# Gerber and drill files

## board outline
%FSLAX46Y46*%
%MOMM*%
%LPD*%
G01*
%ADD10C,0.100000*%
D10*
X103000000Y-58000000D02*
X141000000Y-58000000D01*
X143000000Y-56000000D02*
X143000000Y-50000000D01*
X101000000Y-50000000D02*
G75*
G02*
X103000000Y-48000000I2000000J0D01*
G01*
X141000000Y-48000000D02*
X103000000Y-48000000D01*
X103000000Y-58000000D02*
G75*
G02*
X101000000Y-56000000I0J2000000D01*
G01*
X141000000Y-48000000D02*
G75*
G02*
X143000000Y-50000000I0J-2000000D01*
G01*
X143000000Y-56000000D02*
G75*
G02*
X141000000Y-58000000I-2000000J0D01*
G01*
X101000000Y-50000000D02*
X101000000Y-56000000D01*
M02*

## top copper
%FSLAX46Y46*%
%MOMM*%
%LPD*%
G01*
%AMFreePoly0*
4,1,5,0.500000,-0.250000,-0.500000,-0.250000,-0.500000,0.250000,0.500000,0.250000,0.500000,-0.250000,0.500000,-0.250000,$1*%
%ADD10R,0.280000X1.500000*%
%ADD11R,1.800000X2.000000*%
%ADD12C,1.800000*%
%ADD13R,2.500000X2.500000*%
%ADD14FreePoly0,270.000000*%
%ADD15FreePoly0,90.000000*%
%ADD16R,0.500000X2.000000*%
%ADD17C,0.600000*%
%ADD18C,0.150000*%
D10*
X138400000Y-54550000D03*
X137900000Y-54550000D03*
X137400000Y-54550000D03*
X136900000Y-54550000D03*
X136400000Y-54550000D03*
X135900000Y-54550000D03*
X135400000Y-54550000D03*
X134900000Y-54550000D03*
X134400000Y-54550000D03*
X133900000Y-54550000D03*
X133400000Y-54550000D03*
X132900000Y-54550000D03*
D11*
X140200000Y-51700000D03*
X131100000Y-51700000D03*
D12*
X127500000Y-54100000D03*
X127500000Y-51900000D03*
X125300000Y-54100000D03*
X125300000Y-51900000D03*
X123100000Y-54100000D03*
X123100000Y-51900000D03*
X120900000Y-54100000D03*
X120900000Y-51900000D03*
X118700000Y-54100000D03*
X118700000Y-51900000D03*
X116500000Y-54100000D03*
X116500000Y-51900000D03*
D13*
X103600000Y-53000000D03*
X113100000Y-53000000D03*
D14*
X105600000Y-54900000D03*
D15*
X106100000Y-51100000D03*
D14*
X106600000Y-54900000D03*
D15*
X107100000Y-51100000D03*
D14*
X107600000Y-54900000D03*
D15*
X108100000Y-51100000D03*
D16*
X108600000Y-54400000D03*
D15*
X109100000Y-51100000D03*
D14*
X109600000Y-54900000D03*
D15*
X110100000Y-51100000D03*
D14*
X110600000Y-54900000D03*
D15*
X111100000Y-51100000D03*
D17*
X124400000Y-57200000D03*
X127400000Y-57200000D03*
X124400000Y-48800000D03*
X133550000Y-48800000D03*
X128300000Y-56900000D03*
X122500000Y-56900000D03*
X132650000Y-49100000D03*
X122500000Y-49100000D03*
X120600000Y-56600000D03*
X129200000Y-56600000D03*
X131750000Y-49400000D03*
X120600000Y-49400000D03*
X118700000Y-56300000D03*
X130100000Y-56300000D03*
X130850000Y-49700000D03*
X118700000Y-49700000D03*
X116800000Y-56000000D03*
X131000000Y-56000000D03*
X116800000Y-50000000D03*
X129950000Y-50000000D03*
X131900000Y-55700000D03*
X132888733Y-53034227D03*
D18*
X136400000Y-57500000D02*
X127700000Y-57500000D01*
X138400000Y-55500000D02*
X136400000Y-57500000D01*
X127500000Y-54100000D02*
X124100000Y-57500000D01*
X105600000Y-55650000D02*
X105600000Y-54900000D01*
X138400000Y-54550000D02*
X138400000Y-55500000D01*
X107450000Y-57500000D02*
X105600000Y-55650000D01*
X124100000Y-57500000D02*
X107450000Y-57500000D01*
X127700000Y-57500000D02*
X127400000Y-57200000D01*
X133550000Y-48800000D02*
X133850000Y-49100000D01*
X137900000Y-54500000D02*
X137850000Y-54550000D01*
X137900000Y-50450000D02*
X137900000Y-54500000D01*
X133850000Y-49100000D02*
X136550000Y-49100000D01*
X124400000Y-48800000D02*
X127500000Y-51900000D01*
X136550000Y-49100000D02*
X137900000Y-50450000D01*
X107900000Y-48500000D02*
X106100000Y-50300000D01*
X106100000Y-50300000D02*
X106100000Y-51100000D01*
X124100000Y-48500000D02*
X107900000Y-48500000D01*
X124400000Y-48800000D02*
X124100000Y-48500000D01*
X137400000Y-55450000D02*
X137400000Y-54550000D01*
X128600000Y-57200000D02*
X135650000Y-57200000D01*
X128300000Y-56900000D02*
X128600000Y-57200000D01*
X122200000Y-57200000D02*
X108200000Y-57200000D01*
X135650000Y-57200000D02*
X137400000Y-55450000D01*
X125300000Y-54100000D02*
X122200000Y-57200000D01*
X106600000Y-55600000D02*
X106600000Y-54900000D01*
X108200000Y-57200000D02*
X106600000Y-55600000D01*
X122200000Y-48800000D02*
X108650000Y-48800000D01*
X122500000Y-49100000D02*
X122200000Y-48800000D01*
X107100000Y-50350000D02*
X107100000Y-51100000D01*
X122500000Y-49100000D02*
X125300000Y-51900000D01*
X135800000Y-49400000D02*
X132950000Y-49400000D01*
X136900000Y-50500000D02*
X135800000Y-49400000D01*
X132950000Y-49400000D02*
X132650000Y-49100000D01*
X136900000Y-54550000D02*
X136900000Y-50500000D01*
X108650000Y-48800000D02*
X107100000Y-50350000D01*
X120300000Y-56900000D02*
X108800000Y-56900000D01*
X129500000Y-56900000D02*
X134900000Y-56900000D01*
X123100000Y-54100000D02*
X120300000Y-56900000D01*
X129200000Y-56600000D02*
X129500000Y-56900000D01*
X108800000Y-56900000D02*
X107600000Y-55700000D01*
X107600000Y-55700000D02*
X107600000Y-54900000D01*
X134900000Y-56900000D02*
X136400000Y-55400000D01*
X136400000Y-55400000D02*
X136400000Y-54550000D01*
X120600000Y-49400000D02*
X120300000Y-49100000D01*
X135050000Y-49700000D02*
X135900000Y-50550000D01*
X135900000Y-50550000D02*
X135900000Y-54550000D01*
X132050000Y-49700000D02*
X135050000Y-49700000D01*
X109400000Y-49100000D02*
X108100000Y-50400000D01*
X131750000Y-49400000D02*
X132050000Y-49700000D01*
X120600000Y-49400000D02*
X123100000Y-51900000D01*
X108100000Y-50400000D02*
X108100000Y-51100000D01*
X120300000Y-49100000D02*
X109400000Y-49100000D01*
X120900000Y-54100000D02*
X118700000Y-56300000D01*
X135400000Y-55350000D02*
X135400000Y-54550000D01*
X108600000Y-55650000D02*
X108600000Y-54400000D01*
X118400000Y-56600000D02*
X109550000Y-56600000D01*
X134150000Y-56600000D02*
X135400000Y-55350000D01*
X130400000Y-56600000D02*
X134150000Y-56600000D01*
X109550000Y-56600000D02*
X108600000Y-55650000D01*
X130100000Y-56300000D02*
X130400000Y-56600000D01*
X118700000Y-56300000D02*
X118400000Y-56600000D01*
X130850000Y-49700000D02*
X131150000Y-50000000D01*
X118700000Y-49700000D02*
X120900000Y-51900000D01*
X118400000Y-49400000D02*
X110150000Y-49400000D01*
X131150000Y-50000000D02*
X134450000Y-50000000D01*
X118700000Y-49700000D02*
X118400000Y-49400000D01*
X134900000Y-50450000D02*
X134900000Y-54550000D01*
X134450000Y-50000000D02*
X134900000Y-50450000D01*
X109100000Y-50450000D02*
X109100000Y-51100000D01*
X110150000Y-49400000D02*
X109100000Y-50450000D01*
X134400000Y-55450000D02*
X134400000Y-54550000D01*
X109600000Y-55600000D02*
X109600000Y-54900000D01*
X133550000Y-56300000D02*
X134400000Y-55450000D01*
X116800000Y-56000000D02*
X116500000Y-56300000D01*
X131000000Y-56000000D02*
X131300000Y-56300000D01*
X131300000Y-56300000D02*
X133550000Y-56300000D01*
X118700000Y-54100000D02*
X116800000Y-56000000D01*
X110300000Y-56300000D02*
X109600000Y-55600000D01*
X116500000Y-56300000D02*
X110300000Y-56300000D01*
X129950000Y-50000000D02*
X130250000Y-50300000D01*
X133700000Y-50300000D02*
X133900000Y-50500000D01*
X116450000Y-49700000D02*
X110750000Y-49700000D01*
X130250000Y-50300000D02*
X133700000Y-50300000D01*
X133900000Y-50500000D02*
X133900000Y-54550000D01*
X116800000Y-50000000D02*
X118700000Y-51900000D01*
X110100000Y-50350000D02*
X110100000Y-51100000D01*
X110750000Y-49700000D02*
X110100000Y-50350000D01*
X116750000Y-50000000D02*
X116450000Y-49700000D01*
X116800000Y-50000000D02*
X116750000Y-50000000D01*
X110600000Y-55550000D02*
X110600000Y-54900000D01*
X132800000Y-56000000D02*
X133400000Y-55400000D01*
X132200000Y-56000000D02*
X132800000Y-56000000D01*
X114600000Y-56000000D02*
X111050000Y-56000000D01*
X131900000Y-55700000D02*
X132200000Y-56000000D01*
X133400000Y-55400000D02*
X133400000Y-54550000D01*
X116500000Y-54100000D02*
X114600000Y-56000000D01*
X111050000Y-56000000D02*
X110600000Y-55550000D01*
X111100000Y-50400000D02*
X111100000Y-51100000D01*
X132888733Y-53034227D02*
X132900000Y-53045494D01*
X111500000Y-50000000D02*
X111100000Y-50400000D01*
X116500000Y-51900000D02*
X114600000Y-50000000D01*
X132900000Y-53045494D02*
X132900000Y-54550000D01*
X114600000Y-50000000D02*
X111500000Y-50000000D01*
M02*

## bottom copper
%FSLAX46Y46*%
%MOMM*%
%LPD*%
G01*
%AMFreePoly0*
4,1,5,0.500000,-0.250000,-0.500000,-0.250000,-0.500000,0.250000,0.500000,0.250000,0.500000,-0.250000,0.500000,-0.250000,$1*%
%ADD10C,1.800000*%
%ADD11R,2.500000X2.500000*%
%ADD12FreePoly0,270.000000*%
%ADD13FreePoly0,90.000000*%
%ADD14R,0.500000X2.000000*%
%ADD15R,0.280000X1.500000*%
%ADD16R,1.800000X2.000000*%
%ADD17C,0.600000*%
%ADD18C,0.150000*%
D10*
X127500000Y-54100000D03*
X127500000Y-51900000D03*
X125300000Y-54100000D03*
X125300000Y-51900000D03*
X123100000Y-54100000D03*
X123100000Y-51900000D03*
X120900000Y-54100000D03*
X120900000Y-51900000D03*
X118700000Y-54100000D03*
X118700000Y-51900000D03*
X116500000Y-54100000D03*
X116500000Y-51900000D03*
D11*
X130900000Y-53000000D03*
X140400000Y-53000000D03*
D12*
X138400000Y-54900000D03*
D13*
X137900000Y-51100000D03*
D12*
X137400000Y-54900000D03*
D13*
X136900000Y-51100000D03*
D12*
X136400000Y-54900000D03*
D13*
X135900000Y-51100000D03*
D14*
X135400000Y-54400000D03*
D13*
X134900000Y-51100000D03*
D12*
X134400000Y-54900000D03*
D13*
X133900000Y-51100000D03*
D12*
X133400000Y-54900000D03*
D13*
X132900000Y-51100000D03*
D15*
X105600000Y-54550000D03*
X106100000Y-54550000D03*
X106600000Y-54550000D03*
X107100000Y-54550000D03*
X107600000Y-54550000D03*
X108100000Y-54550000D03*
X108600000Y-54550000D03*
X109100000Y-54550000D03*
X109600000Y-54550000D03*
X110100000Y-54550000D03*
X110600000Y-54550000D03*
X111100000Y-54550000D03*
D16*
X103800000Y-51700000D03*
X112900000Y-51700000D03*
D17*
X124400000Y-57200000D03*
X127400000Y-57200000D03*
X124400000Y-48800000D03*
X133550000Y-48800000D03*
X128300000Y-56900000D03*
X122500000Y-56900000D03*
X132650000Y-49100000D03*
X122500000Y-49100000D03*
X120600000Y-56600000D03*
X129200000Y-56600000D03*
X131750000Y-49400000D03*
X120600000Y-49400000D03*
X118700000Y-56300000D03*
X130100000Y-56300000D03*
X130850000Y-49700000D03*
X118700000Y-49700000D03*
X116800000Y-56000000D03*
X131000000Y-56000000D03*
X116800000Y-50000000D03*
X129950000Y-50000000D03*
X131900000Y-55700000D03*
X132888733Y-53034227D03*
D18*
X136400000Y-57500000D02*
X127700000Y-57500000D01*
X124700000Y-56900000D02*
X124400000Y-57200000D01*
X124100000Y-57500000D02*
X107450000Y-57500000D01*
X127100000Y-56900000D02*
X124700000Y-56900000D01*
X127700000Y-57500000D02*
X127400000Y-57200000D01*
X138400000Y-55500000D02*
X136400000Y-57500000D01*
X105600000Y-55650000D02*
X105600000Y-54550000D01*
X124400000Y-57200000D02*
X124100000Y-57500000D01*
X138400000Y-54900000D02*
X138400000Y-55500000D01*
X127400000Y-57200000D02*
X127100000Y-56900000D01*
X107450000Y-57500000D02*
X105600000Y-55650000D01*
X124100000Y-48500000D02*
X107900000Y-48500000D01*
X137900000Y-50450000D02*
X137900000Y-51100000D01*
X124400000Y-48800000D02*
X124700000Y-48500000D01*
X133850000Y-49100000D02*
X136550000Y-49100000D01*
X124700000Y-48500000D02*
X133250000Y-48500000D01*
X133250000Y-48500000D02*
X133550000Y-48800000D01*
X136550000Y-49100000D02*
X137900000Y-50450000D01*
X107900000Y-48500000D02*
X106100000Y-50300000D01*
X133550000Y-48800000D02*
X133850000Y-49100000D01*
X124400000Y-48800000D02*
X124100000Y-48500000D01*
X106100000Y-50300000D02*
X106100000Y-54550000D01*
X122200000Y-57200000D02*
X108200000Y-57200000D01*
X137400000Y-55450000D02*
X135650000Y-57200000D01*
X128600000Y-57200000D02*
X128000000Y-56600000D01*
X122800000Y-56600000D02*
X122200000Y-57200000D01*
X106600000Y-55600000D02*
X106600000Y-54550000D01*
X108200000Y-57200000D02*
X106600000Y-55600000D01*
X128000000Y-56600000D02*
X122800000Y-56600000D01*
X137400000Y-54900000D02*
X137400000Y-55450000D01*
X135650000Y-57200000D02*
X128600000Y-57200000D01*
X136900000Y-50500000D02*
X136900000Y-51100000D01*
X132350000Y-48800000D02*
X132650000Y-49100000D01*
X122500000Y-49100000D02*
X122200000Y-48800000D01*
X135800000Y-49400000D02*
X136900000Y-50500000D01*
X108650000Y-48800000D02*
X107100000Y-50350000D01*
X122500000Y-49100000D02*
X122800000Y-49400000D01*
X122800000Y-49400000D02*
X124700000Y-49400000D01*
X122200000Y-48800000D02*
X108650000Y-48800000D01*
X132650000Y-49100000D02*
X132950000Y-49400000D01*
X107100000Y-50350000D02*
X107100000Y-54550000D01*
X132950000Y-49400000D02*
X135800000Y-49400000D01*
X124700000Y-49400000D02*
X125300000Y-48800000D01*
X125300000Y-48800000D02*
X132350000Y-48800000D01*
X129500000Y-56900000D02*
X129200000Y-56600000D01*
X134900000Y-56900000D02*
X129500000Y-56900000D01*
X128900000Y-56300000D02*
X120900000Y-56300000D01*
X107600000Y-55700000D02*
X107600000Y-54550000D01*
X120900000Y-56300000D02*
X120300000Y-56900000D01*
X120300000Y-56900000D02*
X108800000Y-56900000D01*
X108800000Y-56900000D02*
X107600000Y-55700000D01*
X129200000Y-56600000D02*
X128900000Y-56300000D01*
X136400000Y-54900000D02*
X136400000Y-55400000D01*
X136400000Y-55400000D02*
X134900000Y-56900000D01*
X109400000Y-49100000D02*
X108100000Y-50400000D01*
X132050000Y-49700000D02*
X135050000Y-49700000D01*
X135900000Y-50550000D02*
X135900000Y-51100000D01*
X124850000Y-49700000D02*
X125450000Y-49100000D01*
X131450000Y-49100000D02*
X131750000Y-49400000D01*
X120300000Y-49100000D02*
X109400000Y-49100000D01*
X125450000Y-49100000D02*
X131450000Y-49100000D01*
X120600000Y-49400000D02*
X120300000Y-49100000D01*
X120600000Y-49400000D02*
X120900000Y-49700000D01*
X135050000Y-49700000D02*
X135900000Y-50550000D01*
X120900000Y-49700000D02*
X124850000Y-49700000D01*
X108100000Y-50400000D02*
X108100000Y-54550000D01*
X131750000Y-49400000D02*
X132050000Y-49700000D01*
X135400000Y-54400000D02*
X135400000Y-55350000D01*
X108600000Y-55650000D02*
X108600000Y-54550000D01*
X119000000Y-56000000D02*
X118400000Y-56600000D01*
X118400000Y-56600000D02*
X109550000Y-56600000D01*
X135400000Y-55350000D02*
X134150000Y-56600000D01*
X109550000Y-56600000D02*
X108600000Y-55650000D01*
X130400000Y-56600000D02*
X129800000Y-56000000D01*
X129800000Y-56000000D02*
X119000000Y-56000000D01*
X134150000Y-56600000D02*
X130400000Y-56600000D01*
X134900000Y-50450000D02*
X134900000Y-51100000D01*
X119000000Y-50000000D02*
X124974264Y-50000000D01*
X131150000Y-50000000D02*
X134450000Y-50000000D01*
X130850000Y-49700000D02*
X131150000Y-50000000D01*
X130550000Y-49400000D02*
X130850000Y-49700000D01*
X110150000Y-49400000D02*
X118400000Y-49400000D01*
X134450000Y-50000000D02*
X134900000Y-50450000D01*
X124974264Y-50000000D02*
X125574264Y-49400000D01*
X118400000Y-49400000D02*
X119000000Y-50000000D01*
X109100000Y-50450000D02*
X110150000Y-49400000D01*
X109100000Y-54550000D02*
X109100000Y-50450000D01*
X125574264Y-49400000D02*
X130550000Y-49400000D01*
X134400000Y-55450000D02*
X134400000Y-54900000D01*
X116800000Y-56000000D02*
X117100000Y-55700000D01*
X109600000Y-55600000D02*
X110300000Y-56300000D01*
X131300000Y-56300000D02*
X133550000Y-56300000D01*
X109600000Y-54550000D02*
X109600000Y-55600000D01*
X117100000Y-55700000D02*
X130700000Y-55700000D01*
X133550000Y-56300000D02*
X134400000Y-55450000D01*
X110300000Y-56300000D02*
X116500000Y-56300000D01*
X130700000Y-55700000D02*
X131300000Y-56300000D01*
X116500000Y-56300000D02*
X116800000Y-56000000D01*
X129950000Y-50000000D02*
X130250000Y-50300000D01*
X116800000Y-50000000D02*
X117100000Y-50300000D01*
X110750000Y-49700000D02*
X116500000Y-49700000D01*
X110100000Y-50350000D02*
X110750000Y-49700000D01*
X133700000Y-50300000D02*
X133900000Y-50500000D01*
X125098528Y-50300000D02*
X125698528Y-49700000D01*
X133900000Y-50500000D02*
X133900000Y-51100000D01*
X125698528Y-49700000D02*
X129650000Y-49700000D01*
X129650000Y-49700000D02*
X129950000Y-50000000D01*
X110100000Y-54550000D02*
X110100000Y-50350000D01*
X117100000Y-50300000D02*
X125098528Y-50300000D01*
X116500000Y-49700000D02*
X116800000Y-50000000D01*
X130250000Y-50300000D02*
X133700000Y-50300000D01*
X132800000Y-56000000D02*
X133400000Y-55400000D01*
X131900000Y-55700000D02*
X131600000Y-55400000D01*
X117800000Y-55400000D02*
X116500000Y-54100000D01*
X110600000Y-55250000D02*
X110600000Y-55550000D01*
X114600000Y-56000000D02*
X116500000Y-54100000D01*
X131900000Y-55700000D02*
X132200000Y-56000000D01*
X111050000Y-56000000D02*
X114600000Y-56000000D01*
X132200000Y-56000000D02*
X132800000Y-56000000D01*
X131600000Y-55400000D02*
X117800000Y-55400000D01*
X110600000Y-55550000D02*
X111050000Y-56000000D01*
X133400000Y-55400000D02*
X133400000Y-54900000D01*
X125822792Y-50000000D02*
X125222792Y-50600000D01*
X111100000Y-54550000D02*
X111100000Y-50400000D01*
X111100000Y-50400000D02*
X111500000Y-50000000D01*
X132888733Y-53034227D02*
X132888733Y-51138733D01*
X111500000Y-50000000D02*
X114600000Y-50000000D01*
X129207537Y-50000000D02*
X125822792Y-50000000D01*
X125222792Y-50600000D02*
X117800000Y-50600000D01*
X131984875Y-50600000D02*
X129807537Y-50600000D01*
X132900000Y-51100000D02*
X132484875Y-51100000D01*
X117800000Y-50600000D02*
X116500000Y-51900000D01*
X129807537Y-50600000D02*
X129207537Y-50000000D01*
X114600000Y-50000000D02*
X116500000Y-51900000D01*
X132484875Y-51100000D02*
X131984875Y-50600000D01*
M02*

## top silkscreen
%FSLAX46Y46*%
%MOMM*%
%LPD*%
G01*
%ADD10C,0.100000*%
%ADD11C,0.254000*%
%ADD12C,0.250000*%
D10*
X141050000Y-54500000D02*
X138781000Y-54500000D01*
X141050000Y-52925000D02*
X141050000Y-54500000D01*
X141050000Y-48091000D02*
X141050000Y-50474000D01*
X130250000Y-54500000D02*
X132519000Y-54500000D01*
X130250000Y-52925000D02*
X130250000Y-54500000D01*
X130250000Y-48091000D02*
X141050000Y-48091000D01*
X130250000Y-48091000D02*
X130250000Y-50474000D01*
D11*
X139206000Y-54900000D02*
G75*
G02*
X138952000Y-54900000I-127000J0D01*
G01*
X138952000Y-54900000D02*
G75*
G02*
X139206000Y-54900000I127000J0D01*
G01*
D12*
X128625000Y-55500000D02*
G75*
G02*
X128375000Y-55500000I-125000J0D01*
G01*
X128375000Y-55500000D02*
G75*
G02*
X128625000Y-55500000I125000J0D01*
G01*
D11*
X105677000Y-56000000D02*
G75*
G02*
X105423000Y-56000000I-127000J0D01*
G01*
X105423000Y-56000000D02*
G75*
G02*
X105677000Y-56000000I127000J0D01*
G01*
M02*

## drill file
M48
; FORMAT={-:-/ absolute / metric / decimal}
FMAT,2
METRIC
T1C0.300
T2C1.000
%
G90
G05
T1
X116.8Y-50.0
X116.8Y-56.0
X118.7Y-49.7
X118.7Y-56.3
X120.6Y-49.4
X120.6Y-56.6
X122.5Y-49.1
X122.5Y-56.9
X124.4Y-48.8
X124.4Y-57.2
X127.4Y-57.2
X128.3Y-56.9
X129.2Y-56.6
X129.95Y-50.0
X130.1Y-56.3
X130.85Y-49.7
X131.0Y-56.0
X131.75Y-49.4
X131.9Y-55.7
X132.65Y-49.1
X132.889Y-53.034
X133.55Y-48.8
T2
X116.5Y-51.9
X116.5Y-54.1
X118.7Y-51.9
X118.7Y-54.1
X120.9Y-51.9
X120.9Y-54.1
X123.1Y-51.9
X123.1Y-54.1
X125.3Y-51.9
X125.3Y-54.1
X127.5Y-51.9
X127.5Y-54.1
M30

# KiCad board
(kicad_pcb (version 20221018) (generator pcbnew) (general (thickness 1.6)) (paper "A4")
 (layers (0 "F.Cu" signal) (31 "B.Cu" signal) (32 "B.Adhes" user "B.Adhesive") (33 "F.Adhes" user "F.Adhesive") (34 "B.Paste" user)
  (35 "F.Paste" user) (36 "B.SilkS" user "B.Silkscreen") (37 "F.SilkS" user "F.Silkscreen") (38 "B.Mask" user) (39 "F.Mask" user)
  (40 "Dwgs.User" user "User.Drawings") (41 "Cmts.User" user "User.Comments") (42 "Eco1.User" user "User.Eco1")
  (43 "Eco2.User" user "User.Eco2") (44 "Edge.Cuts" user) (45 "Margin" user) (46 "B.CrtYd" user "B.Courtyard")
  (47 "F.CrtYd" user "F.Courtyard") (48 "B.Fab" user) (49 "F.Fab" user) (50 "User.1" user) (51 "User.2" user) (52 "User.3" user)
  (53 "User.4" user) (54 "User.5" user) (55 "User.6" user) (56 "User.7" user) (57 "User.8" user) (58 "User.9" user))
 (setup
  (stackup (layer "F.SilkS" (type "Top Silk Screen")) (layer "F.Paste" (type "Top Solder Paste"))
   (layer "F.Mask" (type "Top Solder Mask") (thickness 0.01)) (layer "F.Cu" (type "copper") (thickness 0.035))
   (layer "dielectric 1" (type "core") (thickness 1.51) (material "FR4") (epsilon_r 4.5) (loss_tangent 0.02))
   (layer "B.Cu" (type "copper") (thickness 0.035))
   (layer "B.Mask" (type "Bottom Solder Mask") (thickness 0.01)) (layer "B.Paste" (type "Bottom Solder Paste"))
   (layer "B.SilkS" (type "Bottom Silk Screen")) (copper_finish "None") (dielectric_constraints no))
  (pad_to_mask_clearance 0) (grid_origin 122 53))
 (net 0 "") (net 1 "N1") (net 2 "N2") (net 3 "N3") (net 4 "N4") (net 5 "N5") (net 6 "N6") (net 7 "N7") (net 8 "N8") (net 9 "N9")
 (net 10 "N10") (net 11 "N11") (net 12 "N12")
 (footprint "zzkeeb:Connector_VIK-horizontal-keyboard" (layer "F.Cu") (at 135.65 53 180)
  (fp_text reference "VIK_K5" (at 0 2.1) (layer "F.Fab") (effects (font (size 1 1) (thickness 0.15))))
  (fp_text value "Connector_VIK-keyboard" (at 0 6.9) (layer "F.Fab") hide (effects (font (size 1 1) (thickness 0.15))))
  (fp_line (start -5.4 -1.5) (end -3.131 -1.5) (stroke (width 0.1) (type solid)) (layer "F.SilkS"))
  (fp_line (start -5.4 0.075) (end -5.4 -1.5) (stroke (width 0.1) (type solid)) (layer "F.SilkS"))
  (fp_line (start -5.4 4.909) (end -5.4 2.526) (stroke (width 0.1) (type solid)) (layer "F.SilkS"))
  (fp_line (start 5.4 -1.5) (end 3.131 -1.5) (stroke (width 0.1) (type solid)) (layer "F.SilkS"))
  (fp_line (start 5.4 0.075) (end 5.4 -1.5) (stroke (width 0.1) (type solid)) (layer "F.SilkS"))
  (fp_line (start 5.4 4.909) (end -5.4 4.909) (stroke (width 0.1) (type solid)) (layer "F.SilkS"))
  (fp_line (start 5.4 4.909) (end 5.4 2.526) (stroke (width 0.1) (type solid)) (layer "F.SilkS"))
  (fp_circle (center -3.429 -1.9) (end -3.302 -1.9) (stroke (width 0.254) (type solid)) (fill none) (layer "F.SilkS"))
  (pad "1" smd rect (at -2.75 -1.55 180) (size 0.28 1.5) (layers "F.Cu" "F.Paste" "F.Mask") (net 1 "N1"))
  (pad "2" smd rect (at -2.25 -1.55 180) (size 0.28 1.5) (layers "F.Cu" "F.Paste" "F.Mask") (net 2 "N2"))
  (pad "3" smd rect (at -1.75 -1.55 180) (size 0.28 1.5) (layers "F.Cu" "F.Paste" "F.Mask") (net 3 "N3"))
  (pad "4" smd rect (at -1.25 -1.55 180) (size 0.28 1.5) (layers "F.Cu" "F.Paste" "F.Mask") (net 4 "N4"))
  (pad "5" smd rect (at -0.75 -1.55 180) (size 0.28 1.5) (layers "F.Cu" "F.Paste" "F.Mask") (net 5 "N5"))
  (pad "6" smd rect (at -0.25 -1.55 180) (size 0.28 1.5) (layers "F.Cu" "F.Paste" "F.Mask") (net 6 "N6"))
  (pad "7" smd rect (at 0.25 -1.55 180) (size 0.28 1.5) (layers "F.Cu" "F.Paste" "F.Mask") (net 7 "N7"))
  (pad "8" smd rect (at 0.75 -1.55 180) (size 0.28 1.5) (layers "F.Cu" "F.Paste" "F.Mask") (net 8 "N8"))
  (pad "9" smd rect (at 1.25 -1.55 180) (size 0.28 1.5) (layers "F.Cu" "F.Paste" "F.Mask") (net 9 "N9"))
  (pad "10" smd rect (at 1.75 -1.55 180) (size 0.28 1.5) (layers "F.Cu" "F.Paste" "F.Mask") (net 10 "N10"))
  (pad "11" smd rect (at 2.25 -1.55 180) (size 0.28 1.5) (layers "F.Cu" "F.Paste" "F.Mask") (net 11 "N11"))
  (pad "12" smd rect (at 2.75 -1.55 180) (size 0.28 1.5) (layers "F.Cu" "F.Paste" "F.Mask") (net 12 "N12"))
  (pad "MP" smd rect (at -4.55 1.3 180) (size 1.8 2) (layers "F.Cu" "F.Paste" "F.Mask"))
  (pad "MP" smd rect (at 4.55 1.3 180) (size 1.8 2) (layers "F.Cu" "F.Paste" "F.Mask")))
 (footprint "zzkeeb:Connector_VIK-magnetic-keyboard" (layer "F.Cu") (at 122 53 90)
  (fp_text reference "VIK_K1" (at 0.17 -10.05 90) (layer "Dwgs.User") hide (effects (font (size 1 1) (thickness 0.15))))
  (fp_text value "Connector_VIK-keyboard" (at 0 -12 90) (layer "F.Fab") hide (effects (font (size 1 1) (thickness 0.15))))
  (fp_circle (center -2.5 6.5) (end -2.3 6.5) (stroke (width 0.1) (type solid)) (fill solid) (layer "F.SilkS"))
  (pad "1" thru_hole circle (at -1.1 5.5 270) (size 1.8 1.8) (drill 1) (layers "*.Cu" "*.Mask") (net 1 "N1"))
  (pad "2" thru_hole circle (at 1.1 5.5 270) (size 1.8 1.8) (drill 1) (layers "*.Cu" "*.Mask") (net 2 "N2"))
  (pad "3" thru_hole circle (at -1.1 3.3 270) (size 1.8 1.8) (drill 1) (layers "*.Cu" "*.Mask") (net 3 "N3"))
  (pad "4" thru_hole circle (at 1.1 3.3 270) (size 1.8 1.8) (drill 1) (layers "*.Cu" "*.Mask") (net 4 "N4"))
  (pad "5" thru_hole circle (at -1.1 1.1 270) (size 1.8 1.8) (drill 1) (layers "*.Cu" "*.Mask") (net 5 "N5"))
  (pad "6" thru_hole circle (at 1.1 1.1 270) (size 1.8 1.8) (drill 1) (layers "*.Cu" "*.Mask") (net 6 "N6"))
  (pad "7" thru_hole circle (at -1.1 -1.1 270) (size 1.8 1.8) (drill 1) (layers "*.Cu" "*.Mask") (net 7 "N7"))
  (pad "8" thru_hole circle (at 1.1 -1.1 270) (size 1.8 1.8) (drill 1) (layers "*.Cu" "*.Mask") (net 8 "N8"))
  (pad "9" thru_hole circle (at -1.1 -3.3 270) (size 1.8 1.8) (drill 1) (layers "*.Cu" "*.Mask") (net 9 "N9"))
  (pad "10" thru_hole circle (at 1.1 -3.3 270) (size 1.8 1.8) (drill 1) (layers "*.Cu" "*.Mask") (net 10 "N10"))
  (pad "11" thru_hole circle (at -1.1 -5.5 270) (size 1.8 1.8) (drill 1) (layers "*.Cu" "*.Mask") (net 11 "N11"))
  (pad "12" thru_hole circle (at 1.1 -5.5 270) (size 1.8 1.8) (drill 1) (layers "*.Cu" "*.Mask") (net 12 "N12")))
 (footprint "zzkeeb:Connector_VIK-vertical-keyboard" (layer "F.Cu") (at 108.35 53 90)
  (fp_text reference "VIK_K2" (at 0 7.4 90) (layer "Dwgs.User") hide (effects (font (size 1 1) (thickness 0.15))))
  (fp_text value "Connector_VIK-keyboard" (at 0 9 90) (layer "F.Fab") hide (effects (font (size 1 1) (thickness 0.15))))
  (fp_circle (center -3 -2.8) (end -2.873 -2.8) (stroke (width 0.254) (type solid)) (fill none) (layer "F.SilkS"))
  (pad "" smd rect (at 0 -4.75 90) (size 2.5 2.5) (layers "F.Cu" "F.Paste" "F.Mask"))
  (pad "" smd rect (at 0 4.75 90) (size 2.5 2.5) (layers "F.Cu" "F.Paste" "F.Mask"))
  (pad "1" smd custom (at -1.9 -2.75 270) (size 1 0.5) (layers "F.Cu" "F.Paste" "F.Mask") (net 1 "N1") (thermal_bridge_angle 45)
   (options (clearance outline) (anchor rect)) (primitives))
  (pad "2" smd custom (at 1.9 -2.25 90) (size 1 0.5) (layers "F.Cu" "F.Paste" "F.Mask") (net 2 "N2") (thermal_bridge_angle 45)
   (options (clearance outline) (anchor rect)) (primitives))
  (pad "3" smd custom (at -1.9 -1.75 270) (size 1 0.5) (layers "F.Cu" "F.Paste" "F.Mask") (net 3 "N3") (thermal_bridge_angle 45)
   (options (clearance outline) (anchor rect)) (primitives))
  (pad "4" smd custom (at 1.9 -1.25 90) (size 1 0.5) (layers "F.Cu" "F.Paste" "F.Mask") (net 4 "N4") (thermal_bridge_angle 45)
   (options (clearance outline) (anchor rect)) (primitives))
  (pad "5" smd custom (at -1.9 -0.75 270) (size 1 0.5) (layers "F.Cu" "F.Paste" "F.Mask") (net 5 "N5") (thermal_bridge_angle 45)
   (options (clearance outline) (anchor rect)) (primitives))
  (pad "6" smd custom (at 1.9 -0.25 90) (size 1 0.5) (layers "F.Cu" "F.Paste" "F.Mask") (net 6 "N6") (thermal_bridge_angle 45)
   (options (clearance outline) (anchor rect)) (primitives))
  (pad "7" smd rect (at -1.4 0.25) (size 0.5 2) (layers "F.Cu" "F.Paste" "F.Mask") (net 7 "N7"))
  (pad "8" smd custom (at 1.9 0.75 90) (size 1 0.5) (layers "F.Cu" "F.Paste" "F.Mask") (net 8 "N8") (thermal_bridge_angle 45)
   (options (clearance outline) (anchor rect)) (primitives))
  (pad "9" smd custom (at -1.9 1.25 270) (size 1 0.5) (layers "F.Cu" "F.Paste" "F.Mask") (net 9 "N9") (thermal_bridge_angle 45)
   (options (clearance outline) (anchor rect)) (primitives))
  (pad "10" smd custom (at 1.9 1.75 90) (size 1 0.5) (layers "F.Cu" "F.Paste" "F.Mask") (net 10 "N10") (thermal_bridge_angle 45)
   (options (clearance outline) (anchor rect)) (primitives))
  (pad "11" smd custom (at -1.9 2.25 270) (size 1 0.5) (layers "F.Cu" "F.Paste" "F.Mask") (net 11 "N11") (thermal_bridge_angle 45)
   (options (clearance outline) (anchor rect)) (primitives))
  (pad "12" smd custom (at 1.9 2.75 90) (size 1 0.5) (layers "F.Cu" "F.Paste" "F.Mask") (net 12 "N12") (thermal_bridge_angle 45)
   (options (clearance outline) (anchor rect)) (primitives)))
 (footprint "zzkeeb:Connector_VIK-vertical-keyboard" (layer "B.Cu") (at 135.65 53 90)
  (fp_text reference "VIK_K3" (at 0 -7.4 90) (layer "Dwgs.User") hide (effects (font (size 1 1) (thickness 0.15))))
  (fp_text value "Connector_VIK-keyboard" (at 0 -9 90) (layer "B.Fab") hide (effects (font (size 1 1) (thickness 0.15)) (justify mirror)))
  (pad "" smd rect (at 0 -4.75 90) (size 2.5 2.5) (layers "B.Cu" "B.Paste" "B.Mask"))
  (pad "" smd rect (at 0 4.75 90) (size 2.5 2.5) (layers "B.Cu" "B.Paste" "B.Mask"))
  (pad "1" smd custom (at -1.9 2.75 270) (size 1 0.5) (layers "B.Cu" "B.Paste" "B.Mask") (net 1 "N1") (thermal_bridge_angle 45)
   (options (clearance outline) (anchor rect)) (primitives))
  (pad "2" smd custom (at 1.9 2.25 90) (size 1 0.5) (layers "B.Cu" "B.Paste" "B.Mask") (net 2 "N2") (thermal_bridge_angle 45)
   (options (clearance outline) (anchor rect)) (primitives))
  (pad "3" smd custom (at -1.9 1.75 270) (size 1 0.5) (layers "B.Cu" "B.Paste" "B.Mask") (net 3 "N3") (thermal_bridge_angle 45)
   (options (clearance outline) (anchor rect)) (primitives))
  (pad "4" smd custom (at 1.9 1.25 90) (size 1 0.5) (layers "B.Cu" "B.Paste" "B.Mask") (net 4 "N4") (thermal_bridge_angle 45)
   (options (clearance outline) (anchor rect)) (primitives))
  (pad "5" smd custom (at -1.9 0.75 270) (size 1 0.5) (layers "B.Cu" "B.Paste" "B.Mask") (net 5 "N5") (thermal_bridge_angle 45)
   (options (clearance outline) (anchor rect)) (primitives))
  (pad "6" smd custom (at 1.9 0.25 90) (size 1 0.5) (layers "B.Cu" "B.Paste" "B.Mask") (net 6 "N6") (thermal_bridge_angle 45)
   (options (clearance outline) (anchor rect)) (primitives))
  (pad "7" smd rect (at -1.4 -0.25 180) (size 0.5 2) (layers "B.Cu" "B.Paste" "B.Mask") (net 7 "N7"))
  (pad "8" smd custom (at 1.9 -0.75 90) (size 1 0.5) (layers "B.Cu" "B.Paste" "B.Mask") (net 8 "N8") (thermal_bridge_angle 45)
   (options (clearance outline) (anchor rect)) (primitives))
  (pad "9" smd custom (at -1.9 -1.25 270) (size 1 0.5) (layers "B.Cu" "B.Paste" "B.Mask") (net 9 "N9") (thermal_bridge_angle 45)
   (options (clearance outline) (anchor rect)) (primitives))
  (pad "10" smd custom (at 1.9 -1.75 90) (size 1 0.5) (layers "B.Cu" "B.Paste" "B.Mask") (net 10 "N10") (thermal_bridge_angle 45)
   (options (clearance outline) (anchor rect)) (primitives))
  (pad "11" smd custom (at -1.9 -2.25 270) (size 1 0.5) (layers "B.Cu" "B.Paste" "B.Mask") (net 11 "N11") (thermal_bridge_angle 45)
   (options (clearance outline) (anchor rect)) (primitives))
  (pad "12" smd custom (at 1.9 -2.75 90) (size 1 0.5) (layers "B.Cu" "B.Paste" "B.Mask") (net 12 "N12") (thermal_bridge_angle 45)
   (options (clearance outline) (anchor rect)) (primitives)))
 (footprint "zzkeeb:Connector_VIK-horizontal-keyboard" (layer "B.Cu") (at 108.35 53)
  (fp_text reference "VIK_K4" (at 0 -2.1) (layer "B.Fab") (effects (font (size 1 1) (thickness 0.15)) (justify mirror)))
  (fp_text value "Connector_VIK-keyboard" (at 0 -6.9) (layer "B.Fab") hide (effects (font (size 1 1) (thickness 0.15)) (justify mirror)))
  (pad "1" smd rect (at -2.75 1.55) (size 0.28 1.5) (layers "B.Cu" "B.Paste" "B.Mask") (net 1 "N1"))
  (pad "2" smd rect (at -2.25 1.55) (size 0.28 1.5) (layers "B.Cu" "B.Paste" "B.Mask") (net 2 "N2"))
  (pad "3" smd rect (at -1.75 1.55) (size 0.28 1.5) (layers "B.Cu" "B.Paste" "B.Mask") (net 3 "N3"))
  (pad "4" smd rect (at -1.25 1.55) (size 0.28 1.5) (layers "B.Cu" "B.Paste" "B.Mask") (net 4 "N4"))
  (pad "5" smd rect (at -0.75 1.55) (size 0.28 1.5) (layers "B.Cu" "B.Paste" "B.Mask") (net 5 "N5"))
  (pad "6" smd rect (at -0.25 1.55) (size 0.28 1.5) (layers "B.Cu" "B.Paste" "B.Mask") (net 6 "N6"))
  (pad "7" smd rect (at 0.25 1.55) (size 0.28 1.5) (layers "B.Cu" "B.Paste" "B.Mask") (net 7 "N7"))
  (pad "8" smd rect (at 0.75 1.55) (size 0.28 1.5) (layers "B.Cu" "B.Paste" "B.Mask") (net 8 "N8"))
  (pad "9" smd rect (at 1.25 1.55) (size 0.28 1.5) (layers "B.Cu" "B.Paste" "B.Mask") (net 9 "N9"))
  (pad "10" smd rect (at 1.75 1.55) (size 0.28 1.5) (layers "B.Cu" "B.Paste" "B.Mask") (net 10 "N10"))
  (pad "11" smd rect (at 2.25 1.55) (size 0.28 1.5) (layers "B.Cu" "B.Paste" "B.Mask") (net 11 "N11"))
  (pad "12" smd rect (at 2.75 1.55) (size 0.28 1.5) (layers "B.Cu" "B.Paste" "B.Mask") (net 12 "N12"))
  (pad "MP" smd rect (at -4.55 -1.3) (size 1.8 2) (layers "B.Cu" "B.Paste" "B.Mask"))
  (pad "MP" smd rect (at 4.55 -1.3) (size 1.8 2) (layers "B.Cu" "B.Paste" "B.Mask")))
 (gr_line (start 103 58) (end 141 58) (stroke (width 0.1) (type default)) (layer "Edge.Cuts"))
 (gr_line (start 143 56) (end 143 50) (stroke (width 0.1) (type default)) (layer "Edge.Cuts"))
 (gr_arc (start 101 50) (mid 101.585786 48.585786) (end 103 48) (stroke (width 0.1) (type default)) (layer "Edge.Cuts"))
 (gr_line (start 141 48) (end 103 48) (stroke (width 0.1) (type default)) (layer "Edge.Cuts"))
 (gr_arc (start 103 58) (mid 101.585786 57.414214) (end 101 56) (stroke (width 0.1) (type default)) (layer "Edge.Cuts"))
 (gr_arc (start 141 48) (mid 142.414214 48.585786) (end 143 50) (stroke (width 0.1) (type default)) (layer "Edge.Cuts"))
 (gr_arc (start 143 56) (mid 142.414214 57.414214) (end 141 58) (stroke (width 0.1) (type default)) (layer "Edge.Cuts"))
 (gr_line (start 101 50) (end 101 56) (stroke (width 0.1) (type default)) (layer "Edge.Cuts"))
 (segment (start 136.4 57.5) (end 127.7 57.5) (width 0.15) (layer "F.Cu") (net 1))
 (segment (start 138.4 55.5) (end 136.4 57.5) (width 0.15) (layer "F.Cu") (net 1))
 (segment (start 127.5 54.1) (end 124.1 57.5) (width 0.15) (layer "F.Cu") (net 1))
 (segment (start 105.6 55.65) (end 105.6 54.9) (width 0.15) (layer "F.Cu") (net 1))
 (segment (start 138.4 54.55) (end 138.4 55.5) (width 0.15) (layer "F.Cu") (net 1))
 (segment (start 107.45 57.5) (end 105.6 55.65) (width 0.15) (layer "F.Cu") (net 1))
 (segment (start 124.1 57.5) (end 107.45 57.5) (width 0.15) (layer "F.Cu") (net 1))
 (segment (start 127.7 57.5) (end 127.4 57.2) (width 0.15) (layer "F.Cu") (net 1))
 (via (at 124.4 57.2) (size 0.6) (drill 0.3) (layers "F.Cu" "B.Cu") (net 1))
 (via (at 127.4 57.2) (size 0.6) (drill 0.3) (layers "F.Cu" "B.Cu") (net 1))
 (segment (start 136.4 57.5) (end 127.7 57.5) (width 0.15) (layer "B.Cu") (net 1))
 (segment (start 124.7 56.9) (end 124.4 57.2) (width 0.15) (layer "B.Cu") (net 1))
 (segment (start 124.1 57.5) (end 107.45 57.5) (width 0.15) (layer "B.Cu") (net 1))
 (segment (start 127.1 56.9) (end 124.7 56.9) (width 0.15) (layer "B.Cu") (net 1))
 (segment (start 127.7 57.5) (end 127.4 57.2) (width 0.15) (layer "B.Cu") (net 1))
 (segment (start 138.4 55.5) (end 136.4 57.5) (width 0.15) (layer "B.Cu") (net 1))
 (segment (start 105.6 55.65) (end 105.6 54.55) (width 0.15) (layer "B.Cu") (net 1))
 (segment (start 124.4 57.2) (end 124.1 57.5) (width 0.15) (layer "B.Cu") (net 1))
 (segment (start 138.4 54.9) (end 138.4 55.5) (width 0.15) (layer "B.Cu") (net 1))
 (segment (start 127.4 57.2) (end 127.1 56.9) (width 0.15) (layer "B.Cu") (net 1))
 (segment (start 107.45 57.5) (end 105.6 55.65) (width 0.15) (layer "B.Cu") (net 1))
 (segment (start 133.55 48.8) (end 133.85 49.1) (width 0.15) (layer "F.Cu") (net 2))
 (segment (start 137.9 54.5) (end 137.85 54.55) (width 0.15) (layer "F.Cu") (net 2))
 (segment (start 137.9 50.45) (end 137.9 54.5) (width 0.15) (layer "F.Cu") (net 2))
 (segment (start 133.85 49.1) (end 136.55 49.1) (width 0.15) (layer "F.Cu") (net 2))
 (segment (start 124.4 48.8) (end 127.5 51.9) (width 0.15) (layer "F.Cu") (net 2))
 (segment (start 136.55 49.1) (end 137.9 50.45) (width 0.15) (layer "F.Cu") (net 2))
 (segment (start 107.9 48.5) (end 106.1 50.3) (width 0.15) (layer "F.Cu") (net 2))
 (segment (start 106.1 50.3) (end 106.1 51.1) (width 0.15) (layer "F.Cu") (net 2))
 (segment (start 124.1 48.5) (end 107.9 48.5) (width 0.15) (layer "F.Cu") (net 2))
 (segment (start 124.4 48.8) (end 124.1 48.5) (width 0.15) (layer "F.Cu") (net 2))
 (via locked (at 124.4 48.8) (size 0.6) (drill 0.3) (layers "F.Cu" "B.Cu") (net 2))
 (via locked (at 133.55 48.8) (size 0.6) (drill 0.3) (layers "F.Cu" "B.Cu") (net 2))
 (segment (start 124.1 48.5) (end 107.9 48.5) (width 0.15) (layer "B.Cu") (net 2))
 (segment (start 137.9 50.45) (end 137.9 51.1) (width 0.15) (layer "B.Cu") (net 2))
 (segment (start 124.4 48.8) (end 124.7 48.5) (width 0.15) (layer "B.Cu") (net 2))
 (segment (start 133.85 49.1) (end 136.55 49.1) (width 0.15) (layer "B.Cu") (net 2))
 (segment (start 124.7 48.5) (end 133.25 48.5) (width 0.15) (layer "B.Cu") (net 2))
 (segment (start 133.25 48.5) (end 133.55 48.8) (width 0.15) (layer "B.Cu") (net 2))
 (segment (start 136.55 49.1) (end 137.9 50.45) (width 0.15) (layer "B.Cu") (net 2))
 (segment (start 107.9 48.5) (end 106.1 50.3) (width 0.15) (layer "B.Cu") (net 2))
 (segment (start 133.55 48.8) (end 133.85 49.1) (width 0.15) (layer "B.Cu") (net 2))
 (segment (start 124.4 48.8) (end 124.1 48.5) (width 0.15) (layer "B.Cu") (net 2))
 (segment (start 106.1 50.3) (end 106.1 54.55) (width 0.15) (layer "B.Cu") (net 2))
 (segment (start 137.4 55.45) (end 137.4 54.55) (width 0.15) (layer "F.Cu") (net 3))
 (segment (start 128.6 57.2) (end 135.65 57.2) (width 0.15) (layer "F.Cu") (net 3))
 (segment (start 128.3 56.9) (end 128.6 57.2) (width 0.15) (layer "F.Cu") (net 3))
 (segment (start 122.2 57.2) (end 108.2 57.2) (width 0.15) (layer "F.Cu") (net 3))
 (segment (start 135.65 57.2) (end 137.4 55.45) (width 0.15) (layer "F.Cu") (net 3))
 (segment (start 125.3 54.1) (end 122.2 57.2) (width 0.15) (layer "F.Cu") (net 3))
 (segment (start 106.6 55.6) (end 106.6 54.9) (width 0.15) (layer "F.Cu") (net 3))
 (segment (start 108.2 57.2) (end 106.6 55.6) (width 0.15) (layer "F.Cu") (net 3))
 (via (at 128.3 56.9) (size 0.6) (drill 0.3) (layers "F.Cu" "B.Cu") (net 3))
 (via (at 122.5 56.9) (size 0.6) (drill 0.3) (layers "F.Cu" "B.Cu") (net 3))
 (segment (start 122.2 57.2) (end 108.2 57.2) (width 0.15) (layer "B.Cu") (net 3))
 (segment (start 137.4 55.45) (end 135.65 57.2) (width 0.15) (layer "B.Cu") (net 3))
 (segment (start 128.6 57.2) (end 128 56.6) (width 0.15) (layer "B.Cu") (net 3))
 (segment (start 122.8 56.6) (end 122.2 57.2) (width 0.15) (layer "B.Cu") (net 3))
 (segment (start 106.6 55.6) (end 106.6 54.55) (width 0.15) (layer "B.Cu") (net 3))
 (segment (start 108.2 57.2) (end 106.6 55.6) (width 0.15) (layer "B.Cu") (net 3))
 (segment (start 128 56.6) (end 122.8 56.6) (width 0.15) (layer "B.Cu") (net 3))
 (segment (start 137.4 54.9) (end 137.4 55.45) (width 0.15) (layer "B.Cu") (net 3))
 (segment (start 135.65 57.2) (end 128.6 57.2) (width 0.15) (layer "B.Cu") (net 3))
 (segment (start 122.2 48.8) (end 108.65 48.8) (width 0.15) (layer "F.Cu") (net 4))
 (segment (start 122.5 49.1) (end 122.2 48.8) (width 0.15) (layer "F.Cu") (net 4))
 (segment (start 107.1 50.35) (end 107.1 51.1) (width 0.15) (layer "F.Cu") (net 4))
 (segment (start 122.5 49.1) (end 125.3 51.9) (width 0.15) (layer "F.Cu") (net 4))
 (segment (start 135.8 49.4) (end 132.95 49.4) (width 0.15) (layer "F.Cu") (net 4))
 (segment (start 136.9 50.5) (end 135.8 49.4) (width 0.15) (layer "F.Cu") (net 4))
 (segment (start 132.95 49.4) (end 132.65 49.1) (width 0.15) (layer "F.Cu") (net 4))
 (segment (start 136.9 54.55) (end 136.9 50.5) (width 0.15) (layer "F.Cu") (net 4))
 (segment (start 108.65 48.8) (end 107.1 50.35) (width 0.15) (layer "F.Cu") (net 4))
 (via locked (at 132.65 49.1) (size 0.6) (drill 0.3) (layers "F.Cu" "B.Cu") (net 4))
 (via locked (at 122.5 49.1) (size 0.6) (drill 0.3) (layers "F.Cu" "B.Cu") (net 4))
 (segment (start 136.9 50.5) (end 136.9 51.1) (width 0.15) (layer "B.Cu") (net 4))
 (segment (start 132.35 48.8) (end 132.65 49.1) (width 0.15) (layer "B.Cu") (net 4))
 (segment (start 122.5 49.1) (end 122.2 48.8) (width 0.15) (layer "B.Cu") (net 4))
 (segment (start 135.8 49.4) (end 136.9 50.5) (width 0.15) (layer "B.Cu") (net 4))
 (segment (start 108.65 48.8) (end 107.1 50.35) (width 0.15) (layer "B.Cu") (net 4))
 (segment (start 122.5 49.1) (end 122.8 49.4) (width 0.15) (layer "B.Cu") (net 4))
 (segment (start 122.8 49.4) (end 124.7 49.4) (width 0.15) (layer "B.Cu") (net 4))
 (segment (start 122.2 48.8) (end 108.65 48.8) (width 0.15) (layer "B.Cu") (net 4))
 (segment (start 132.65 49.1) (end 132.95 49.4) (width 0.15) (layer "B.Cu") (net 4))
 (segment (start 107.1 50.35) (end 107.1 54.55) (width 0.15) (layer "B.Cu") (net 4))
 (segment (start 132.95 49.4) (end 135.8 49.4) (width 0.15) (layer "B.Cu") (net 4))
 (segment (start 124.7 49.4) (end 125.3 48.8) (width 0.15) (layer "B.Cu") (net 4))
 (segment (start 125.3 48.8) (end 132.35 48.8) (width 0.15) (layer "B.Cu") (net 4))
 (segment (start 120.3 56.9) (end 108.8 56.9) (width 0.15) (layer "F.Cu") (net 5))
 (segment (start 129.5 56.9) (end 134.9 56.9) (width 0.15) (layer "F.Cu") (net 5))
 (segment (start 123.1 54.1) (end 120.3 56.9) (width 0.15) (layer "F.Cu") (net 5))
 (segment (start 129.2 56.6) (end 129.5 56.9) (width 0.15) (layer "F.Cu") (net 5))
 (segment (start 108.8 56.9) (end 107.6 55.7) (width 0.15) (layer "F.Cu") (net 5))
 (segment (start 107.6 55.7) (end 107.6 54.9) (width 0.15) (layer "F.Cu") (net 5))
 (segment (start 134.9 56.9) (end 136.4 55.4) (width 0.15) (layer "F.Cu") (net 5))
 (segment (start 136.4 55.4) (end 136.4 54.55) (width 0.15) (layer "F.Cu") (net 5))
 (via locked (at 120.6 56.6) (size 0.6) (drill 0.3) (layers "F.Cu" "B.Cu") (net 5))
 (via (at 129.2 56.6) (size 0.6) (drill 0.3) (layers "F.Cu" "B.Cu") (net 5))
 (segment (start 129.5 56.9) (end 129.2 56.6) (width 0.15) (layer "B.Cu") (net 5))
 (segment (start 134.9 56.9) (end 129.5 56.9) (width 0.15) (layer "B.Cu") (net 5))
 (segment (start 128.9 56.3) (end 120.9 56.3) (width 0.15) (layer "B.Cu") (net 5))
 (segment (start 107.6 55.7) (end 107.6 54.55) (width 0.15) (layer "B.Cu") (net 5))
 (segment (start 120.9 56.3) (end 120.3 56.9) (width 0.15) (layer "B.Cu") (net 5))
 (segment (start 120.3 56.9) (end 108.8 56.9) (width 0.15) (layer "B.Cu") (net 5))
 (segment (start 108.8 56.9) (end 107.6 55.7) (width 0.15) (layer "B.Cu") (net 5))
 (segment (start 129.2 56.6) (end 128.9 56.3) (width 0.15) (layer "B.Cu") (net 5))
 (segment (start 136.4 54.9) (end 136.4 55.4) (width 0.15) (layer "B.Cu") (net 5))
 (segment (start 136.4 55.4) (end 134.9 56.9) (width 0.15) (layer "B.Cu") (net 5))
 (segment (start 120.6 49.4) (end 120.3 49.1) (width 0.15) (layer "F.Cu") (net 6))
 (segment (start 135.05 49.7) (end 135.9 50.55) (width 0.15) (layer "F.Cu") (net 6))
 (segment (start 135.9 50.55) (end 135.9 54.55) (width 0.15) (layer "F.Cu") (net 6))
 (segment (start 132.05 49.7) (end 135.05 49.7) (width 0.15) (layer "F.Cu") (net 6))
 (segment (start 109.4 49.1) (end 108.1 50.4) (width 0.15) (layer "F.Cu") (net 6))
 (segment (start 131.75 49.4) (end 132.05 49.7) (width 0.15) (layer "F.Cu") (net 6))
 (segment (start 120.6 49.4) (end 123.1 51.9) (width 0.15) (layer "F.Cu") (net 6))
 (segment (start 108.1 50.4) (end 108.1 51.1) (width 0.15) (layer "F.Cu") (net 6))
 (segment (start 120.3 49.1) (end 109.4 49.1) (width 0.15) (layer "F.Cu") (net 6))
 (via locked (at 131.75 49.4) (size 0.6) (drill 0.3) (layers "F.Cu" "B.Cu") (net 6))
 (via locked (at 120.6 49.4) (size 0.6) (drill 0.3) (layers "F.Cu" "B.Cu") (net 6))
 (segment (start 109.4 49.1) (end 108.1 50.4) (width 0.15) (layer "B.Cu") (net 6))
 (segment (start 132.05 49.7) (end 135.05 49.7) (width 0.15) (layer "B.Cu") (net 6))
 (segment (start 135.9 50.55) (end 135.9 51.1) (width 0.15) (layer "B.Cu") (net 6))
 (segment (start 124.85 49.7) (end 125.45 49.1) (width 0.15) (layer "B.Cu") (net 6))
 (segment (start 131.45 49.1) (end 131.75 49.4) (width 0.15) (layer "B.Cu") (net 6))
 (segment (start 120.3 49.1) (end 109.4 49.1) (width 0.15) (layer "B.Cu") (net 6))
 (segment (start 125.45 49.1) (end 131.45 49.1) (width 0.15) (layer "B.Cu") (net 6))
 (segment (start 120.6 49.4) (end 120.3 49.1) (width 0.15) (layer "B.Cu") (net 6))
 (segment (start 120.6 49.4) (end 120.9 49.7) (width 0.15) (layer "B.Cu") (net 6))
 (segment (start 135.05 49.7) (end 135.9 50.55) (width 0.15) (layer "B.Cu") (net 6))
 (segment (start 120.9 49.7) (end 124.85 49.7) (width 0.15) (layer "B.Cu") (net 6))
 (segment (start 108.1 50.4) (end 108.1 54.55) (width 0.15) (layer "B.Cu") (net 6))
 (segment (start 131.75 49.4) (end 132.05 49.7) (width 0.15) (layer "B.Cu") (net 6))
 (segment (start 120.9 54.1) (end 118.7 56.3) (width 0.15) (layer "F.Cu") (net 7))
 (segment (start 135.4 55.35) (end 135.4 54.55) (width 0.15) (layer "F.Cu") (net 7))
 (segment (start 108.6 55.65) (end 108.6 54.4) (width 0.15) (layer "F.Cu") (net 7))
 (segment (start 118.4 56.6) (end 109.55 56.6) (width 0.15) (layer "F.Cu") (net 7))
 (segment (start 134.15 56.6) (end 135.4 55.35) (width 0.15) (layer "F.Cu") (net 7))
 (segment (start 130.4 56.6) (end 134.15 56.6) (width 0.15) (layer "F.Cu") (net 7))
 (segment (start 109.55 56.6) (end 108.6 55.65) (width 0.15) (layer "F.Cu") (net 7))
 (segment (start 130.1 56.3) (end 130.4 56.6) (width 0.15) (layer "F.Cu") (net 7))
 (segment (start 118.7 56.3) (end 118.4 56.6) (width 0.15) (layer "F.Cu") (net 7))
 (via locked (at 118.7 56.3) (size 0.6) (drill 0.3) (layers "F.Cu" "B.Cu") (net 7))
 (via (at 130.1 56.3) (size 0.6) (drill 0.3) (layers "F.Cu" "B.Cu") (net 7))
 (segment (start 135.4 54.4) (end 135.4 55.35) (width 0.15) (layer "B.Cu") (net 7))
 (segment (start 108.6 55.65) (end 108.6 54.55) (width 0.15) (layer "B.Cu") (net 7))
 (segment (start 119 56) (end 118.4 56.6) (width 0.15) (layer "B.Cu") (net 7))
 (segment (start 118.4 56.6) (end 109.55 56.6) (width 0.15) (layer "B.Cu") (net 7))
 (segment (start 135.4 55.35) (end 134.15 56.6) (width 0.15) (layer "B.Cu") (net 7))
 (segment (start 109.55 56.6) (end 108.6 55.65) (width 0.15) (layer "B.Cu") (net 7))
 (segment (start 130.4 56.6) (end 129.8 56) (width 0.15) (layer "B.Cu") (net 7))
 (segment (start 129.8 56) (end 119 56) (width 0.15) (layer "B.Cu") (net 7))
 (segment (start 134.15 56.6) (end 130.4 56.6) (width 0.15) (layer "B.Cu") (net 7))
 (segment (start 130.85 49.7) (end 131.15 50) (width 0.15) (layer "F.Cu") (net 8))
 (segment (start 118.7 49.7) (end 120.9 51.9) (width 0.15) (layer "F.Cu") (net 8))
 (segment (start 118.4 49.4) (end 110.15 49.4) (width 0.15) (layer "F.Cu") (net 8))
 (segment (start 131.15 50) (end 134.45 50) (width 0.15) (layer "F.Cu") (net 8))
 (segment (start 118.7 49.7) (end 118.4 49.4) (width 0.15) (layer "F.Cu") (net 8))
 (segment (start 134.9 50.45) (end 134.9 54.55) (width 0.15) (layer "F.Cu") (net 8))
 (segment (start 134.45 50) (end 134.9 50.45) (width 0.15) (layer "F.Cu") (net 8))
 (segment (start 109.1 50.45) (end 109.1 51.1) (width 0.15) (layer "F.Cu") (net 8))
 (segment (start 110.15 49.4) (end 109.1 50.45) (width 0.15) (layer "F.Cu") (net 8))
 (via locked (at 130.85 49.7) (size 0.6) (drill 0.3) (layers "F.Cu" "B.Cu") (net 8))
 (via locked (at 118.7 49.7) (size 0.6) (drill 0.3) (layers "F.Cu" "B.Cu") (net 8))
 (segment (start 134.9 50.45) (end 134.9 51.1) (width 0.15) (layer "B.Cu") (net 8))
 (segment (start 119 50) (end 124.974264 50) (width 0.15) (layer "B.Cu") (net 8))
 (segment (start 131.15 50) (end 134.45 50) (width 0.15) (layer "B.Cu") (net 8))
 (segment (start 130.85 49.7) (end 131.15 50) (width 0.15) (layer "B.Cu") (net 8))
 (segment (start 130.55 49.4) (end 130.85 49.7) (width 0.15) (layer "B.Cu") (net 8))
 (segment (start 110.15 49.4) (end 118.4 49.4) (width 0.15) (layer "B.Cu") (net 8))
 (segment (start 134.45 50) (end 134.9 50.45) (width 0.15) (layer "B.Cu") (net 8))
 (segment (start 124.974264 50) (end 125.574264 49.4) (width 0.15) (layer "B.Cu") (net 8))
 (segment (start 118.4 49.4) (end 119 50) (width 0.15) (layer "B.Cu") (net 8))
 (segment (start 109.1 50.45) (end 110.15 49.4) (width 0.15) (layer "B.Cu") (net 8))
 (segment (start 109.1 54.55) (end 109.1 50.45) (width 0.15) (layer "B.Cu") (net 8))
 (segment (start 125.574264 49.4) (end 130.55 49.4) (width 0.15) (layer "B.Cu") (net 8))
 (segment (start 134.4 55.45) (end 134.4 54.55) (width 0.15) (layer "F.Cu") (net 9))
 (segment (start 109.6 55.6) (end 109.6 54.9) (width 0.15) (layer "F.Cu") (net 9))
 (segment (start 133.55 56.3) (end 134.4 55.45) (width 0.15) (layer "F.Cu") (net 9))
 (segment (start 116.8 56) (end 116.5 56.3) (width 0.15) (layer "F.Cu") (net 9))
 (segment (start 131 56) (end 131.3 56.3) (width 0.15) (layer "F.Cu") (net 9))
 (segment (start 131.3 56.3) (end 133.55 56.3) (width 0.15) (layer "F.Cu") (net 9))
 (segment (start 118.7 54.1) (end 116.8 56) (width 0.15) (layer "F.Cu") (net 9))
 (segment (start 110.3 56.3) (end 109.6 55.6) (width 0.15) (layer "F.Cu") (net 9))
 (segment (start 116.5 56.3) (end 110.3 56.3) (width 0.15) (layer "F.Cu") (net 9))
 (via locked (at 116.8 56) (size 0.6) (drill 0.3) (layers "F.Cu" "B.Cu") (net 9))
 (via (at 131 56) (size 0.6) (drill 0.3) (layers "F.Cu" "B.Cu") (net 9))
 (segment (start 134.4 55.45) (end 134.4 54.9) (width 0.15) (layer "B.Cu") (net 9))
 (segment (start 116.8 56) (end 117.1 55.7) (width 0.15) (layer "B.Cu") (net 9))
 (segment (start 109.6 55.6) (end 110.3 56.3) (width 0.15) (layer "B.Cu") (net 9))
 (segment (start 131.3 56.3) (end 133.55 56.3) (width 0.15) (layer "B.Cu") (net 9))
 (segment (start 109.6 54.55) (end 109.6 55.6) (width 0.15) (layer "B.Cu") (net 9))
 (segment (start 117.1 55.7) (end 130.7 55.7) (width 0.15) (layer "B.Cu") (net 9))
 (segment (start 133.55 56.3) (end 134.4 55.45) (width 0.15) (layer "B.Cu") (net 9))
 (segment (start 110.3 56.3) (end 116.5 56.3) (width 0.15) (layer "B.Cu") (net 9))
 (segment (start 130.7 55.7) (end 131.3 56.3) (width 0.15) (layer "B.Cu") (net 9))
 (segment (start 116.5 56.3) (end 116.8 56) (width 0.15) (layer "B.Cu") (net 9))
 (segment (start 129.95 50) (end 130.25 50.3) (width 0.15) (layer "F.Cu") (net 10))
 (segment (start 133.7 50.3) (end 133.9 50.5) (width 0.15) (layer "F.Cu") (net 10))
 (segment (start 116.45 49.7) (end 110.75 49.7) (width 0.15) (layer "F.Cu") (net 10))
 (segment (start 130.25 50.3) (end 133.7 50.3) (width 0.15) (layer "F.Cu") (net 10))
 (segment (start 133.9 50.5) (end 133.9 54.55) (width 0.15) (layer "F.Cu") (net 10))
 (segment (start 116.8 50) (end 118.7 51.9) (width 0.15) (layer "F.Cu") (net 10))
 (segment (start 110.1 50.35) (end 110.1 51.1) (width 0.15) (layer "F.Cu") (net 10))
 (segment (start 110.75 49.7) (end 110.1 50.35) (width 0.15) (layer "F.Cu") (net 10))
 (segment (start 116.75 50) (end 116.45 49.7) (width 0.15) (layer "F.Cu") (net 10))
 (segment (start 116.8 50) (end 116.75 50) (width 0.15) (layer "F.Cu") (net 10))
 (via locked (at 116.8 50) (size 0.6) (drill 0.3) (layers "F.Cu" "B.Cu") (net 10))
 (via locked (at 129.95 50) (size 0.6) (drill 0.3) (layers "F.Cu" "B.Cu") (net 10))
 (segment (start 129.95 50) (end 130.25 50.3) (width 0.15) (layer "B.Cu") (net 10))
 (segment (start 116.8 50) (end 117.1 50.3) (width 0.15) (layer "B.Cu") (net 10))
 (segment (start 110.75 49.7) (end 116.5 49.7) (width 0.15) (layer "B.Cu") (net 10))
 (segment (start 110.1 50.35) (end 110.75 49.7) (width 0.15) (layer "B.Cu") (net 10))
 (segment (start 133.7 50.3) (end 133.9 50.5) (width 0.15) (layer "B.Cu") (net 10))
 (segment (start 125.098528 50.3) (end 125.698528 49.7) (width 0.15) (layer "B.Cu") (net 10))
 (segment (start 133.9 50.5) (end 133.9 51.1) (width 0.15) (layer "B.Cu") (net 10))
 (segment (start 125.698528 49.7) (end 129.65 49.7) (width 0.15) (layer "B.Cu") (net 10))
 (segment (start 129.65 49.7) (end 129.95 50) (width 0.15) (layer "B.Cu") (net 10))
 (segment (start 110.1 54.55) (end 110.1 50.35) (width 0.15) (layer "B.Cu") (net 10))
 (segment (start 117.1 50.3) (end 125.098528 50.3) (width 0.15) (layer "B.Cu") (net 10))
 (segment (start 116.5 49.7) (end 116.8 50) (width 0.15) (layer "B.Cu") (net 10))
 (segment (start 130.25 50.3) (end 133.7 50.3) (width 0.15) (layer "B.Cu") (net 10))
 (segment (start 110.6 55.55) (end 110.6 54.9) (width 0.15) (layer "F.Cu") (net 11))
 (segment (start 132.8 56) (end 133.4 55.4) (width 0.15) (layer "F.Cu") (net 11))
 (segment (start 132.2 56) (end 132.8 56) (width 0.15) (layer "F.Cu") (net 11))
 (segment (start 114.6 56) (end 111.05 56) (width 0.15) (layer "F.Cu") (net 11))
 (segment (start 131.9 55.7) (end 132.2 56) (width 0.15) (layer "F.Cu") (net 11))
 (segment (start 133.4 55.4) (end 133.4 54.55) (width 0.15) (layer "F.Cu") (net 11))
 (segment (start 116.5 54.1) (end 114.6 56) (width 0.15) (layer "F.Cu") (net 11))
 (segment (start 111.05 56) (end 110.6 55.55) (width 0.15) (layer "F.Cu") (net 11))
 (via (at 131.9 55.7) (size 0.6) (drill 0.3) (layers "F.Cu" "B.Cu") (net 11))
 (segment (start 132.8 56) (end 133.4 55.4) (width 0.15) (layer "B.Cu") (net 11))
 (segment (start 131.9 55.7) (end 131.6 55.4) (width 0.15) (layer "B.Cu") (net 11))
 (segment (start 117.8 55.4) (end 116.5 54.1) (width 0.15) (layer "B.Cu") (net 11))
 (segment (start 110.6 55.25) (end 110.6 55.55) (width 0.15) (layer "B.Cu") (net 11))
 (segment (start 114.6 56) (end 116.5 54.1) (width 0.15) (layer "B.Cu") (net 11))
 (segment (start 131.9 55.7) (end 132.2 56) (width 0.15) (layer "B.Cu") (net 11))
 (segment (start 111.05 56) (end 114.6 56) (width 0.15) (layer "B.Cu") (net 11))
 (segment (start 132.2 56) (end 132.8 56) (width 0.15) (layer "B.Cu") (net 11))
 (segment (start 131.6 55.4) (end 117.8 55.4) (width 0.15) (layer "B.Cu") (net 11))
 (segment (start 110.6 55.55) (end 111.05 56) (width 0.15) (layer "B.Cu") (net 11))
 (segment (start 133.4 55.4) (end 133.4 54.9) (width 0.15) (layer "B.Cu") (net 11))
 (segment (start 111.1 50.4) (end 111.1 51.1) (width 0.15) (layer "F.Cu") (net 12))
 (segment (start 132.888733 53.034227) (end 132.9 53.045494) (width 0.15) (layer "F.Cu") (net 12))
 (segment (start 111.5 50) (end 111.1 50.4) (width 0.15) (layer "F.Cu") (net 12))
 (segment (start 116.5 51.9) (end 114.6 50) (width 0.15) (layer "F.Cu") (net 12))
 (segment (start 132.9 53.045494) (end 132.9 54.55) (width 0.15) (layer "F.Cu") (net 12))
 (segment (start 114.6 50) (end 111.5 50) (width 0.15) (layer "F.Cu") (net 12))
 (via (at 132.888733 53.034227) (size 0.6) (drill 0.3) (layers "F.Cu" "B.Cu") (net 12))
 (segment (start 125.822792 50) (end 125.222792 50.6) (width 0.15) (layer "B.Cu") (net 12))
 (segment (start 111.1 54.55) (end 111.1 50.4) (width 0.15) (layer "B.Cu") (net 12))
 (segment (start 111.1 50.4) (end 111.5 50) (width 0.15) (layer "B.Cu") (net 12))
 (segment (start 132.888733 53.034227) (end 132.888733 51.138733) (width 0.15) (layer "B.Cu") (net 12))
 (segment (start 111.5 50) (end 114.6 50) (width 0.15) (layer "B.Cu") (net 12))
 (segment (start 129.207537 50) (end 125.822792 50) (width 0.15) (layer "B.Cu") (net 12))
 (segment (start 125.222792 50.6) (end 117.8 50.6) (width 0.15) (layer "B.Cu") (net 12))
 (segment (start 131.984875 50.6) (end 129.807537 50.6) (width 0.15) (layer "B.Cu") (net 12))
 (segment (start 132.9 51.1) (end 132.484875 51.1) (width 0.15) (layer "B.Cu") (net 12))
 (segment (start 117.8 50.6) (end 116.5 51.9) (width 0.15) (layer "B.Cu") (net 12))
 (segment (start 129.807537 50.6) (end 129.207537 50) (width 0.15) (layer "B.Cu") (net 12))
 (segment (start 114.6 50) (end 116.5 51.9) (width 0.15) (layer "B.Cu") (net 12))
 (segment (start 132.484875 51.1) (end 131.984875 50.6) (width 0.15) (layer "B.Cu") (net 12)))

